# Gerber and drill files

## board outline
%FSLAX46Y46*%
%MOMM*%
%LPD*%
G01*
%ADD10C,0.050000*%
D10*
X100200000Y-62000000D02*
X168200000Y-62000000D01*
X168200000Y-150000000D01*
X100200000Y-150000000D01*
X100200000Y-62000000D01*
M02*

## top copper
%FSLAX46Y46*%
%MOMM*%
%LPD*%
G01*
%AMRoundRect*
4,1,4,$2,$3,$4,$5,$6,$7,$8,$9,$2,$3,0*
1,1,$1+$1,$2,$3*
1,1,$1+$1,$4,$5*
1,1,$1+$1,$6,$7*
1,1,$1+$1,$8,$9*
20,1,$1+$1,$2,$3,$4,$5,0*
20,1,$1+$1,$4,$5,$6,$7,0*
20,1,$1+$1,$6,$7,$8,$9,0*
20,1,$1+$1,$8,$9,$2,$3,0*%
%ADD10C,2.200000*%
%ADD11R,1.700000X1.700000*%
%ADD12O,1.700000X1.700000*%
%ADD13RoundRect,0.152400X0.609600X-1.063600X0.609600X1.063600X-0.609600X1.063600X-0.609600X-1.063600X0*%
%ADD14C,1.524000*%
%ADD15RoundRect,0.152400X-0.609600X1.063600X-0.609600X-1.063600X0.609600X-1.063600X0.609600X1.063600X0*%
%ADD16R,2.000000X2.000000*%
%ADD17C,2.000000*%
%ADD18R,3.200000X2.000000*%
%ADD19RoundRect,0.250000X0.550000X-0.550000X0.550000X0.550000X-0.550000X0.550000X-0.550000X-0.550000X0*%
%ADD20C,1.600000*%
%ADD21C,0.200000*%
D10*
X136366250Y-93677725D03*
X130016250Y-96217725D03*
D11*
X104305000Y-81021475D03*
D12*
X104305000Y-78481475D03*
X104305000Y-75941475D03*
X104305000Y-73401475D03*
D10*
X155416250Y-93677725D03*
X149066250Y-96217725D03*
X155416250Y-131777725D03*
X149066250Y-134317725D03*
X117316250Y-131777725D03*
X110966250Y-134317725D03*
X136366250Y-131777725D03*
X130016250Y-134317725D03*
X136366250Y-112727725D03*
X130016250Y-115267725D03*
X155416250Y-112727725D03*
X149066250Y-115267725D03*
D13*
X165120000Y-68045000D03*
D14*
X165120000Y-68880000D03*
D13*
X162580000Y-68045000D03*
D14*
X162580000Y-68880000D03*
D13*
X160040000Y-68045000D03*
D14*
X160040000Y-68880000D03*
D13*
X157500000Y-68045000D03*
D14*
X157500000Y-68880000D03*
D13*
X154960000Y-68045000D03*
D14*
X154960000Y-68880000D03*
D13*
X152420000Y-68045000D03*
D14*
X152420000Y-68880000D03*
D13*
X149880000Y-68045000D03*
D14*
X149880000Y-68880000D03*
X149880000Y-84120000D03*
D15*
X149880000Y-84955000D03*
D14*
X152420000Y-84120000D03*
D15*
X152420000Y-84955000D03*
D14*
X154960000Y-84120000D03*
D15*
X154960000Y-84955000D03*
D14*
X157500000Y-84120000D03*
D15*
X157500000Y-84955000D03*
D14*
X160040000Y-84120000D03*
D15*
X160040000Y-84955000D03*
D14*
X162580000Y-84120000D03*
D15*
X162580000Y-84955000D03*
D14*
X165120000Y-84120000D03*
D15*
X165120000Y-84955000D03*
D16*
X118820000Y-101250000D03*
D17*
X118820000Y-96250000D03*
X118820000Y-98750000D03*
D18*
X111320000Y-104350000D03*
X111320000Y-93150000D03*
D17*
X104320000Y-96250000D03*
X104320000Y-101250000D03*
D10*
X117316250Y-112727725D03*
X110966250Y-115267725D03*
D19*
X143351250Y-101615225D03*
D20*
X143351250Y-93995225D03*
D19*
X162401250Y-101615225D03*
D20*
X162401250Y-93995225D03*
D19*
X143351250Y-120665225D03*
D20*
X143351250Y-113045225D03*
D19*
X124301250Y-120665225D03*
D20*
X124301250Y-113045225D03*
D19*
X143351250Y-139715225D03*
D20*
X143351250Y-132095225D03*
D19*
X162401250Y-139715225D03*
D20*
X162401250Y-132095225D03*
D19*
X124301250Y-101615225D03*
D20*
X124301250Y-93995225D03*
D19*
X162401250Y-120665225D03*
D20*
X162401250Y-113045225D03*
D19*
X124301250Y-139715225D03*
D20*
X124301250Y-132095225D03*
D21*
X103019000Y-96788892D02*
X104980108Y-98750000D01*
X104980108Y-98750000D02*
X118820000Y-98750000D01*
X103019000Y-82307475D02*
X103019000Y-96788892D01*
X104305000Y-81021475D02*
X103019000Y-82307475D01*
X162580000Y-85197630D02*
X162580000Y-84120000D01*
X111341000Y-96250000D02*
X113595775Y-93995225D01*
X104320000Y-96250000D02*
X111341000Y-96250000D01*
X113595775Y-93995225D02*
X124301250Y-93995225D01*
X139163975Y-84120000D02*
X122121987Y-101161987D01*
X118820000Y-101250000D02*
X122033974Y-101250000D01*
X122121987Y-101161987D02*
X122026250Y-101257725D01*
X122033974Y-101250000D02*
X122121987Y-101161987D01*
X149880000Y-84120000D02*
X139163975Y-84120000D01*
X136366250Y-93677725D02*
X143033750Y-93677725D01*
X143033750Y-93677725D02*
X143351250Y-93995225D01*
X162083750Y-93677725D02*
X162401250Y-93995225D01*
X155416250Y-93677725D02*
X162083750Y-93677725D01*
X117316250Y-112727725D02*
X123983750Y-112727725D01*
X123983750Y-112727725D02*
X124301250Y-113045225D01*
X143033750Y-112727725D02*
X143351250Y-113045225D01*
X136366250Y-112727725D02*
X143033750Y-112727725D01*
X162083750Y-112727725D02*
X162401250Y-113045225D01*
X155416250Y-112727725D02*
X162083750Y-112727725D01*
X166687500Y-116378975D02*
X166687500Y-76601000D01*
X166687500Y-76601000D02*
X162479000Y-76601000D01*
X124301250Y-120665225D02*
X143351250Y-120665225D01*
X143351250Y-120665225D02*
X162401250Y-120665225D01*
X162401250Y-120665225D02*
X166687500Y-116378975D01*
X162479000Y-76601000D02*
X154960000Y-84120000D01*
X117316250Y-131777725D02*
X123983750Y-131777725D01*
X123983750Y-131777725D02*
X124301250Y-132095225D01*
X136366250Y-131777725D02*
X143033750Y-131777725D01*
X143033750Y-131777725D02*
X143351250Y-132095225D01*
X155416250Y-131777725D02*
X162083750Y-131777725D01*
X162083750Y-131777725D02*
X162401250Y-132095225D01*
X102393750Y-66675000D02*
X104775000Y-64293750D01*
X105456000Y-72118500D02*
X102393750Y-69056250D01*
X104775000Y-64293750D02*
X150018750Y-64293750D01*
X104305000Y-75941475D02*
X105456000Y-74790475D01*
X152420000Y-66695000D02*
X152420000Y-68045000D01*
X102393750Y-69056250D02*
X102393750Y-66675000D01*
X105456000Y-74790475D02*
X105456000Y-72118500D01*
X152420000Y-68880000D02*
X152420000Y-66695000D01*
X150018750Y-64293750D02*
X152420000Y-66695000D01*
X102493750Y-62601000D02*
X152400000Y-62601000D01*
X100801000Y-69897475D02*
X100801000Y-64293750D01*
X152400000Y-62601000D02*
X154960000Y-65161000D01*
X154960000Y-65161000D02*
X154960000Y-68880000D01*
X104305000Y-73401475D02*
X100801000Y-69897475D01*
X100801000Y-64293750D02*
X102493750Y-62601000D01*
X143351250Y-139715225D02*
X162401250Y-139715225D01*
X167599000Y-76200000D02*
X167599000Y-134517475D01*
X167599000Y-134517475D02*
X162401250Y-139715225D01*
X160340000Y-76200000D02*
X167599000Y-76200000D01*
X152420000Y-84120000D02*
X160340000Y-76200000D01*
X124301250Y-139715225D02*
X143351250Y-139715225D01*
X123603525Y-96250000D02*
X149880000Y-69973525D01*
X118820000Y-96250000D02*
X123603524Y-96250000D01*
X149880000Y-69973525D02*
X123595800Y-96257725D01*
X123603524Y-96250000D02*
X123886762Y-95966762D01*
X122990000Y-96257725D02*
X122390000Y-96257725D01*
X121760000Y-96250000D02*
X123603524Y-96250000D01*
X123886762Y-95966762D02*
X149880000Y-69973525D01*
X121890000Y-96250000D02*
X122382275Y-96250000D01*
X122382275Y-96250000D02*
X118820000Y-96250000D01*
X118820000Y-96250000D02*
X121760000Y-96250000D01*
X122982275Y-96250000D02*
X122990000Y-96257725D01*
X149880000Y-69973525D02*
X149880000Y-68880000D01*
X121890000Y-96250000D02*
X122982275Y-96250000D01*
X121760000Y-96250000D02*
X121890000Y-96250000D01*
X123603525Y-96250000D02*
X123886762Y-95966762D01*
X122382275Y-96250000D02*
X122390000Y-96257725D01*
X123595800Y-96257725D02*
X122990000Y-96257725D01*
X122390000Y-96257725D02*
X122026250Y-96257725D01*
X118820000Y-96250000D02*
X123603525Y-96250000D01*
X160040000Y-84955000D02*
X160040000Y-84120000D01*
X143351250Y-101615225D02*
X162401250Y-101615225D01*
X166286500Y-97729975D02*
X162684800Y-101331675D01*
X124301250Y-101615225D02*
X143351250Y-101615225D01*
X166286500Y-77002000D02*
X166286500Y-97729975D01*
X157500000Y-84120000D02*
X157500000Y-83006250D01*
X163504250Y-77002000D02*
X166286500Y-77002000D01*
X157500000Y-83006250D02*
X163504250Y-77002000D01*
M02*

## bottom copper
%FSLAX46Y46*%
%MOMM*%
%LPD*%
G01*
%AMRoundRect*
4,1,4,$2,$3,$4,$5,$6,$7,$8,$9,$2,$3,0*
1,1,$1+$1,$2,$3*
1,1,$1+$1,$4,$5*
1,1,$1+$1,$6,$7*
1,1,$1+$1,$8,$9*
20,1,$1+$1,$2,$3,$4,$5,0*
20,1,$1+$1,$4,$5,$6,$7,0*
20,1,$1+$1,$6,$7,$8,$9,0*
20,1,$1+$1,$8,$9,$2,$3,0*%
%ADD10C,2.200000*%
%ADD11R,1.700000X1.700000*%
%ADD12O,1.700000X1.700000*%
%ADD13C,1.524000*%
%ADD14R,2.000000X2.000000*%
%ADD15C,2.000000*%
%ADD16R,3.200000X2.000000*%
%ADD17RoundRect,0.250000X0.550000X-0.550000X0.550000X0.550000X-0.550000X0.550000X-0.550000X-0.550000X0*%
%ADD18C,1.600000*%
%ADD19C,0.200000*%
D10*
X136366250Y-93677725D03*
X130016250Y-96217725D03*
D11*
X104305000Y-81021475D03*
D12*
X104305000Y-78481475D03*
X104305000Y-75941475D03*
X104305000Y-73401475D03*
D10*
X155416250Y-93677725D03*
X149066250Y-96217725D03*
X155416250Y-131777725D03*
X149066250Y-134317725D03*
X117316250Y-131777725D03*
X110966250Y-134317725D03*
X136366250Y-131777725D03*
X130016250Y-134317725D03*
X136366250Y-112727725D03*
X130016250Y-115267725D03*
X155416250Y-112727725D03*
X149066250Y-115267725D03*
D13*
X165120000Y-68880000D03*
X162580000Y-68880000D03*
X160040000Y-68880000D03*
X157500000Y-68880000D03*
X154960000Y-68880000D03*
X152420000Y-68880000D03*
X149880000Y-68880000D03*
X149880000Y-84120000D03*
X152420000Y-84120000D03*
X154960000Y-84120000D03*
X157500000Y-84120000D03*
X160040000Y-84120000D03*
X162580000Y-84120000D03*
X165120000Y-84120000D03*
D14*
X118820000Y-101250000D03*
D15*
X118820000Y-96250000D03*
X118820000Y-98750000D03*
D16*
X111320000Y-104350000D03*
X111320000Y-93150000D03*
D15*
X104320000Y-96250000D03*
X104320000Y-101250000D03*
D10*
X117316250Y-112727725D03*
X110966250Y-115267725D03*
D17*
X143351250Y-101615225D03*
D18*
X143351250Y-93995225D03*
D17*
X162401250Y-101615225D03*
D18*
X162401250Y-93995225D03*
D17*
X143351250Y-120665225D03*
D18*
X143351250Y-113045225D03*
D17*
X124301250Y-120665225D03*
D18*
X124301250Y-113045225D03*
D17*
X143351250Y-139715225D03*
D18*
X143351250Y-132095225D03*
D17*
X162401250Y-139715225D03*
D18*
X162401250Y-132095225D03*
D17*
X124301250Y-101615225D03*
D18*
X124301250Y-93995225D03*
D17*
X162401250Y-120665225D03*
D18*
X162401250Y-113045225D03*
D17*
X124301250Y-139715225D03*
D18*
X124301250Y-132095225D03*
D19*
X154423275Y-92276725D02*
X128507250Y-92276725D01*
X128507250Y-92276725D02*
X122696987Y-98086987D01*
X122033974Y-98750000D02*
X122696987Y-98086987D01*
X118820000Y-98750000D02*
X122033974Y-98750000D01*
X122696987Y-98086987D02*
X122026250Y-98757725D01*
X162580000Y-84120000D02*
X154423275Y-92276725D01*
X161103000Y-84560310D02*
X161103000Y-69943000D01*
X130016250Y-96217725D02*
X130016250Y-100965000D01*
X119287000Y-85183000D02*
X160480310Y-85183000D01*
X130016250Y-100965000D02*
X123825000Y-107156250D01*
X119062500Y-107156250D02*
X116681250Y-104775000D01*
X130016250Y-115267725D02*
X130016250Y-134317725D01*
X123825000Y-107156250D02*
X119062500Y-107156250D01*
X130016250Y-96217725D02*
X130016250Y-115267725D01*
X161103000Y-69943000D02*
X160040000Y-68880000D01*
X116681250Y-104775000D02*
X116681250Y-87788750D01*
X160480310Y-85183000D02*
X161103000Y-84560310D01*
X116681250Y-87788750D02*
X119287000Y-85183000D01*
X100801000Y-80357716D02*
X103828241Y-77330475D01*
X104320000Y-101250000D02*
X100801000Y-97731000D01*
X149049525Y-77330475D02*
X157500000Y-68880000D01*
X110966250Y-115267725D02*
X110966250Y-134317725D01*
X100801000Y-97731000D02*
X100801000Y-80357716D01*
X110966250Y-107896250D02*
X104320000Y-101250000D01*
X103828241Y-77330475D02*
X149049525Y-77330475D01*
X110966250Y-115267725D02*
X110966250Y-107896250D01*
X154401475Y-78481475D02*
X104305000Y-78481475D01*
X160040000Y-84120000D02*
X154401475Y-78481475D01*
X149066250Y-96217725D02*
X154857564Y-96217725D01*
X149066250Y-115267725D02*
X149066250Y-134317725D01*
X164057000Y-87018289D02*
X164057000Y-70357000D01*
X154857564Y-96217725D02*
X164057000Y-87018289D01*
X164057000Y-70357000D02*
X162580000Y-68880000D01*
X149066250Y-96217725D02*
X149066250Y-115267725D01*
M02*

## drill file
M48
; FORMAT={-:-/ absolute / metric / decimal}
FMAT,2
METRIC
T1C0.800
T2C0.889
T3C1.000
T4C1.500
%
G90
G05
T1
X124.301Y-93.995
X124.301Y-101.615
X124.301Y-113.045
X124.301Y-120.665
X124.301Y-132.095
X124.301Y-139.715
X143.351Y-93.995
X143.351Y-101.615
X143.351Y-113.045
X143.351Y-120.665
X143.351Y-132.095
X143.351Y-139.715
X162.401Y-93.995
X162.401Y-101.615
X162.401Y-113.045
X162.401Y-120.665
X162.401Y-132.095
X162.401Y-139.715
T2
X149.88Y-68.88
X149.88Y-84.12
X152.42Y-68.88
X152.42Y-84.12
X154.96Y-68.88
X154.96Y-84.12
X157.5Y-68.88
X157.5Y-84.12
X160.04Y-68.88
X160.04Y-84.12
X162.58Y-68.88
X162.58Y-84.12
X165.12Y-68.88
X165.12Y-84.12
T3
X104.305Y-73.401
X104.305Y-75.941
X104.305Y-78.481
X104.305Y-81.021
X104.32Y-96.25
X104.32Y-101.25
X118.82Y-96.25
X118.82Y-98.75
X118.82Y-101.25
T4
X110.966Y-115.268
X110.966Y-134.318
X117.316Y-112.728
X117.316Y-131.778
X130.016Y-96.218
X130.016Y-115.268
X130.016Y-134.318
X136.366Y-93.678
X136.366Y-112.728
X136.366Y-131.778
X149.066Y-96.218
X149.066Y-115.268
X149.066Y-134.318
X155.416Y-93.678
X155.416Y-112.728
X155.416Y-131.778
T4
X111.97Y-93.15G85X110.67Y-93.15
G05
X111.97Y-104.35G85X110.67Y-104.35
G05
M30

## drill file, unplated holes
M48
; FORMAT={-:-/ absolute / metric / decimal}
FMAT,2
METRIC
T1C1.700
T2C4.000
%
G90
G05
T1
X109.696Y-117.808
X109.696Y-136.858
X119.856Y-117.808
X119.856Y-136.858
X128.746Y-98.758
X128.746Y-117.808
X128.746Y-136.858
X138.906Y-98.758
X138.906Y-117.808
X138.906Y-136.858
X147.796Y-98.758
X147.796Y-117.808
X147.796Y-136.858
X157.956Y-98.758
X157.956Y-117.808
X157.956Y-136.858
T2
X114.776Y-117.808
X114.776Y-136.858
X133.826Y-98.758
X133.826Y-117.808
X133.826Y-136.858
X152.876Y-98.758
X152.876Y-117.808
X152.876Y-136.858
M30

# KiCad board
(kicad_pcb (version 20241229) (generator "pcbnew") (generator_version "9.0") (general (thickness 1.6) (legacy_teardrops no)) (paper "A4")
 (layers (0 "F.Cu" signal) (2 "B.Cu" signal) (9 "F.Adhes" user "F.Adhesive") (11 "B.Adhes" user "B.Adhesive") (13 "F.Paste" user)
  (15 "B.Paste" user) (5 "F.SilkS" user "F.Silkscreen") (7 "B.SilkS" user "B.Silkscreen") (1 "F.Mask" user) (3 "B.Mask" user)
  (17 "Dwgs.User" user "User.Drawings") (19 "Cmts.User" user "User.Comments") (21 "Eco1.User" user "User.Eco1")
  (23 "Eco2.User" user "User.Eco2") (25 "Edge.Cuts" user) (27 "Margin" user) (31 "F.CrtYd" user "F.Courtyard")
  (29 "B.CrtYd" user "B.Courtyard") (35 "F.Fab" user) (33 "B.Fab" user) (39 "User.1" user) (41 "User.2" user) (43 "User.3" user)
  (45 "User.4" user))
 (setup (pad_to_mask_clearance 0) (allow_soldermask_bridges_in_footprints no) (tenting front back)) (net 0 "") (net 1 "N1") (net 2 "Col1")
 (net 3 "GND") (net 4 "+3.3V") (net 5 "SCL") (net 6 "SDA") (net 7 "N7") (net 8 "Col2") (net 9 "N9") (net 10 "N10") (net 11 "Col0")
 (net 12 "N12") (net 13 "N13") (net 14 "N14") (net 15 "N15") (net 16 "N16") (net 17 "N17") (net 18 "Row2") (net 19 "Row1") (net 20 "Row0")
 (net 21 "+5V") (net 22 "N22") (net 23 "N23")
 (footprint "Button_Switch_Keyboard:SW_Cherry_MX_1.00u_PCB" (layer "F.Cu") (at 136.36625 93.677725)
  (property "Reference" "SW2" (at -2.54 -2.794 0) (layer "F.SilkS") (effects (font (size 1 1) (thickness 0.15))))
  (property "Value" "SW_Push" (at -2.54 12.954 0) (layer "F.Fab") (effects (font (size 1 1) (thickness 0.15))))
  (pad "" np_thru_hole circle (at -7.62 5.08) (size 1.7 1.7) (drill 1.7) (layers "*.Cu" "*.Mask"))
  (pad "" np_thru_hole circle (at -2.54 5.08) (size 4 4) (drill 4) (layers "*.Cu" "*.Mask"))
  (pad "" np_thru_hole circle (at 2.54 5.08) (size 1.7 1.7) (drill 1.7) (layers "*.Cu" "*.Mask"))
  (pad "1" thru_hole circle (at 0 0) (size 2.2 2.2) (drill 1.5) (layers "*.Cu" "*.Mask") (remove_unused_layers no) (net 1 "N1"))
  (pad "2" thru_hole circle (at -6.35 2.54) (size 2.2 2.2) (drill 1.5) (layers "*.Cu" "*.Mask") (remove_unused_layers no) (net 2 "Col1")))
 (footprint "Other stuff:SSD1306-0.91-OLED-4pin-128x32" (layer "F.Cu") (at 140.805 83.211475 180)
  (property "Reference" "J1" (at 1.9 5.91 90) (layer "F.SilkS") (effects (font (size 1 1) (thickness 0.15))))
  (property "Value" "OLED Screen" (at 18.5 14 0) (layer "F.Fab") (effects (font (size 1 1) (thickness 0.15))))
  (pad "1" thru_hole rect (at 36.5 2.19 180) (size 1.7 1.7) (drill 1) (layers "*.Cu" "*.Mask") (remove_unused_layers no) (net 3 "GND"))
  (pad "2" thru_hole oval (at 36.5 4.73 180) (size 1.7 1.7) (drill 1) (layers "*.Cu" "*.Mask") (remove_unused_layers no) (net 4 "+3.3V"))
  (pad "3" thru_hole oval (at 36.5 7.27 180) (size 1.7 1.7) (drill 1) (layers "*.Cu" "*.Mask") (remove_unused_layers no) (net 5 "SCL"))
  (pad "4" thru_hole oval (at 36.5 9.81 180) (size 1.7 1.7) (drill 1) (layers "*.Cu" "*.Mask") (remove_unused_layers no) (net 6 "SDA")))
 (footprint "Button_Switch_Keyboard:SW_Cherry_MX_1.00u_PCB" (layer "F.Cu") (at 155.41625 93.677725)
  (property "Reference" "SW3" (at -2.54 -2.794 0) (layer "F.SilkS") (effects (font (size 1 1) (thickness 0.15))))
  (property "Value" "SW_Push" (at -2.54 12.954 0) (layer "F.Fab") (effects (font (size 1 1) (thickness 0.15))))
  (pad "" np_thru_hole circle (at -7.62 5.08) (size 1.7 1.7) (drill 1.7) (layers "*.Cu" "*.Mask"))
  (pad "" np_thru_hole circle (at -2.54 5.08) (size 4 4) (drill 4) (layers "*.Cu" "*.Mask"))
  (pad "" np_thru_hole circle (at 2.54 5.08) (size 1.7 1.7) (drill 1.7) (layers "*.Cu" "*.Mask"))
  (pad "1" thru_hole circle (at 0 0) (size 2.2 2.2) (drill 1.5) (layers "*.Cu" "*.Mask") (remove_unused_layers no) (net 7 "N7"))
  (pad "2" thru_hole circle (at -6.35 2.54) (size 2.2 2.2) (drill 1.5) (layers "*.Cu" "*.Mask") (remove_unused_layers no) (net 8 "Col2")))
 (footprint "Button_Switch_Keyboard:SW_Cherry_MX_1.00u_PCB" (layer "F.Cu") (at 155.41625 131.777725)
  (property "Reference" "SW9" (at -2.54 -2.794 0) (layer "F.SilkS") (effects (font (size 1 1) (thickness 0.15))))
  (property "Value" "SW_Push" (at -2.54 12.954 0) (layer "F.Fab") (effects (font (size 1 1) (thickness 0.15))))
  (pad "" np_thru_hole circle (at -7.62 5.08) (size 1.7 1.7) (drill 1.7) (layers "*.Cu" "*.Mask"))
  (pad "" np_thru_hole circle (at -2.54 5.08) (size 4 4) (drill 4) (layers "*.Cu" "*.Mask"))
  (pad "" np_thru_hole circle (at 2.54 5.08) (size 1.7 1.7) (drill 1.7) (layers "*.Cu" "*.Mask"))
  (pad "1" thru_hole circle (at 0 0) (size 2.2 2.2) (drill 1.5) (layers "*.Cu" "*.Mask") (remove_unused_layers no) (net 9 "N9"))
  (pad "2" thru_hole circle (at -6.35 2.54) (size 2.2 2.2) (drill 1.5) (layers "*.Cu" "*.Mask") (remove_unused_layers no) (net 8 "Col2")))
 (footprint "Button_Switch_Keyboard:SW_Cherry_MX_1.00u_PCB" (layer "F.Cu") (at 117.31625 131.777725)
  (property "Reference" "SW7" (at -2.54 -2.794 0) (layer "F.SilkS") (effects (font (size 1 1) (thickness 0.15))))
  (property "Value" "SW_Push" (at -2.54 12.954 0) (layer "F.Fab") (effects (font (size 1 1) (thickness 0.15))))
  (pad "" np_thru_hole circle (at -7.62 5.08) (size 1.7 1.7) (drill 1.7) (layers "*.Cu" "*.Mask"))
  (pad "" np_thru_hole circle (at -2.54 5.08) (size 4 4) (drill 4) (layers "*.Cu" "*.Mask"))
  (pad "" np_thru_hole circle (at 2.54 5.08) (size 1.7 1.7) (drill 1.7) (layers "*.Cu" "*.Mask"))
  (pad "1" thru_hole circle (at 0 0) (size 2.2 2.2) (drill 1.5) (layers "*.Cu" "*.Mask") (remove_unused_layers no) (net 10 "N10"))
  (pad "2" thru_hole circle (at -6.35 2.54) (size 2.2 2.2) (drill 1.5) (layers "*.Cu" "*.Mask") (remove_unused_layers no) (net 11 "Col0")))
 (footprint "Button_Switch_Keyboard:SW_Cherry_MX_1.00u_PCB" (layer "F.Cu") (at 136.36625 131.777725)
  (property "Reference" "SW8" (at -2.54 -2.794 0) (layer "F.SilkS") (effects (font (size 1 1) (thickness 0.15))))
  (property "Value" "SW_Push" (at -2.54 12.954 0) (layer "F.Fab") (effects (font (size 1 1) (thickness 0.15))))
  (pad "" np_thru_hole circle (at -7.62 5.08) (size 1.7 1.7) (drill 1.7) (layers "*.Cu" "*.Mask"))
  (pad "" np_thru_hole circle (at -2.54 5.08) (size 4 4) (drill 4) (layers "*.Cu" "*.Mask"))
  (pad "" np_thru_hole circle (at 2.54 5.08) (size 1.7 1.7) (drill 1.7) (layers "*.Cu" "*.Mask"))
  (pad "1" thru_hole circle (at 0 0) (size 2.2 2.2) (drill 1.5) (layers "*.Cu" "*.Mask") (remove_unused_layers no) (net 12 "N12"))
  (pad "2" thru_hole circle (at -6.35 2.54) (size 2.2 2.2) (drill 1.5) (layers "*.Cu" "*.Mask") (remove_unused_layers no) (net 2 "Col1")))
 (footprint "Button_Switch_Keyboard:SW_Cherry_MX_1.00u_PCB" (layer "F.Cu") (at 136.36625 112.727725)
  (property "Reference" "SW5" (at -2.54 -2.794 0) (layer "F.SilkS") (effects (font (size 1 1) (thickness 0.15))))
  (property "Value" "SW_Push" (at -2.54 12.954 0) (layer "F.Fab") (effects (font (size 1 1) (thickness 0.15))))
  (pad "" np_thru_hole circle (at -7.62 5.08) (size 1.7 1.7) (drill 1.7) (layers "*.Cu" "*.Mask"))
  (pad "" np_thru_hole circle (at -2.54 5.08) (size 4 4) (drill 4) (layers "*.Cu" "*.Mask"))
  (pad "" np_thru_hole circle (at 2.54 5.08) (size 1.7 1.7) (drill 1.7) (layers "*.Cu" "*.Mask"))
  (pad "1" thru_hole circle (at 0 0) (size 2.2 2.2) (drill 1.5) (layers "*.Cu" "*.Mask") (remove_unused_layers no) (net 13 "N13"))
  (pad "2" thru_hole circle (at -6.35 2.54) (size 2.2 2.2) (drill 1.5) (layers "*.Cu" "*.Mask") (remove_unused_layers no) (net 2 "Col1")))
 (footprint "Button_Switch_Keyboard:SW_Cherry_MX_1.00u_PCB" (layer "F.Cu") (at 155.41625 112.727725)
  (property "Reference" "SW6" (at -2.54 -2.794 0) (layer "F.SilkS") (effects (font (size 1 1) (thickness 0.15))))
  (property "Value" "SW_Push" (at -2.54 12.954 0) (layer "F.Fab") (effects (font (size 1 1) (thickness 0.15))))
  (pad "" np_thru_hole circle (at -7.62 5.08) (size 1.7 1.7) (drill 1.7) (layers "*.Cu" "*.Mask"))
  (pad "" np_thru_hole circle (at -2.54 5.08) (size 4 4) (drill 4) (layers "*.Cu" "*.Mask"))
  (pad "" np_thru_hole circle (at 2.54 5.08) (size 1.7 1.7) (drill 1.7) (layers "*.Cu" "*.Mask"))
  (pad "1" thru_hole circle (at 0 0) (size 2.2 2.2) (drill 1.5) (layers "*.Cu" "*.Mask") (remove_unused_layers no) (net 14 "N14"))
  (pad "2" thru_hole circle (at -6.35 2.54) (size 2.2 2.2) (drill 1.5) (layers "*.Cu" "*.Mask") (remove_unused_layers no) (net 8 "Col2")))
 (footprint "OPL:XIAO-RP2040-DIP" (layer "F.Cu") (at 157.5 76.5 -90)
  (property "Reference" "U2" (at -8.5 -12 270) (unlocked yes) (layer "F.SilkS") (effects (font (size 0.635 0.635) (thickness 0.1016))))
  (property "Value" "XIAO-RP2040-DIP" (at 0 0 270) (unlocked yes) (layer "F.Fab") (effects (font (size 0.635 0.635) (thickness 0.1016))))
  (pad "1" smd roundrect (at -8.455 -7.62 90) (size 2.432 1.524) (layers "F.Cu" "F.Mask") (roundrect_rratio 0.1) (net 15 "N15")
   (thermal_bridge_angle 45))
  (pad "1" thru_hole circle (at -7.62 -7.62 90) (size 1.524 1.524) (drill 0.889) (layers "*.Cu" "*.Mask") (remove_unused_layers no)
   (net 15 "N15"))
  (pad "2" smd roundrect (at -8.455 -5.08 90) (size 2.432 1.524) (layers "F.Cu" "F.Mask") (roundrect_rratio 0.1) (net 8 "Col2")
   (thermal_bridge_angle 45))
  (pad "2" thru_hole circle (at -7.62 -5.08 90) (size 1.524 1.524) (drill 0.889) (layers "*.Cu" "*.Mask") (remove_unused_layers no)
   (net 8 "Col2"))
  (pad "3" smd roundrect (at -8.455 -2.54 90) (size 2.432 1.524) (layers "F.Cu" "F.Mask") (roundrect_rratio 0.1) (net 2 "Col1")
   (thermal_bridge_angle 45))
  (pad "3" thru_hole circle (at -7.62 -2.54 90) (size 1.524 1.524) (drill 0.889) (layers "*.Cu" "*.Mask") (remove_unused_layers no)
   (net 2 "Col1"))
  (pad "4" smd roundrect (at -8.455 0 90) (size 2.432 1.524) (layers "F.Cu" "F.Mask") (roundrect_rratio 0.1) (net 11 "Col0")
   (thermal_bridge_angle 45))
  (pad "4" thru_hole circle (at -7.62 0 90) (size 1.524 1.524) (drill 0.889) (layers "*.Cu" "*.Mask") (remove_unused_layers no)
   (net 11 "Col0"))
  (pad "5" smd roundrect (at -8.455 2.54 90) (size 2.432 1.524) (layers "F.Cu" "F.Mask") (roundrect_rratio 0.1) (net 6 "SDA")
   (thermal_bridge_angle 45))
  (pad "5" thru_hole circle (at -7.62 2.54 90) (size 1.524 1.524) (drill 0.889) (layers "*.Cu" "*.Mask") (remove_unused_layers no)
   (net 6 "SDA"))
  (pad "6" smd roundrect (at -8.455 5.08 90) (size 2.432 1.524) (layers "F.Cu" "F.Mask") (roundrect_rratio 0.1) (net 5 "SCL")
   (thermal_bridge_angle 45))
  (pad "6" thru_hole circle (at -7.62 5.08 90) (size 1.524 1.524) (drill 0.889) (layers "*.Cu" "*.Mask") (remove_unused_layers no)
   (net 5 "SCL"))
  (pad "7" smd roundrect (at -8.455 7.62 90) (size 2.432 1.524) (layers "F.Cu" "F.Mask") (roundrect_rratio 0.1) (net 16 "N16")
   (thermal_bridge_angle 45))
  (pad "7" thru_hole circle (at -7.62 7.62 90) (size 1.524 1.524) (drill 0.889) (layers "*.Cu" "*.Mask") (remove_unused_layers no)
   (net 16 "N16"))
  (pad "8" thru_hole circle (at 7.62 7.62 270) (size 1.524 1.524) (drill 0.889) (layers "*.Cu" "*.Mask") (remove_unused_layers no)
   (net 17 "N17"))
  (pad "8" smd roundrect (at 8.455 7.62 270) (size 2.432 1.524) (layers "F.Cu" "F.Mask") (roundrect_rratio 0.1) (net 17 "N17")
   (thermal_bridge_angle 45))
  (pad "9" thru_hole circle (at 7.62 5.08 270) (size 1.524 1.524) (drill 0.889) (layers "*.Cu" "*.Mask") (remove_unused_layers no)
   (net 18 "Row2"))
  (pad "9" smd roundrect (at 8.455 5.08 270) (size 2.432 1.524) (layers "F.Cu" "F.Mask") (roundrect_rratio 0.1) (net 18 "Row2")
   (thermal_bridge_angle 45))
  (pad "10" thru_hole circle (at 7.62 2.54 270) (size 1.524 1.524) (drill 0.889) (layers "*.Cu" "*.Mask") (remove_unused_layers no)
   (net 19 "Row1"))
  (pad "10" smd roundrect (at 8.455 2.54 270) (size 2.432 1.524) (layers "F.Cu" "F.Mask") (roundrect_rratio 0.1) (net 19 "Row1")
   (thermal_bridge_angle 45))
  (pad "11" thru_hole circle (at 7.62 0 270) (size 1.524 1.524) (drill 0.889) (layers "*.Cu" "*.Mask") (remove_unused_layers no)
   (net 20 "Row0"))
  (pad "11" smd roundrect (at 8.455 0 270) (size 2.432 1.524) (layers "F.Cu" "F.Mask") (roundrect_rratio 0.1) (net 20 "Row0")
   (thermal_bridge_angle 45))
  (pad "12" thru_hole circle (at 7.62 -2.54 270) (size 1.524 1.524) (drill 0.889) (layers "*.Cu" "*.Mask") (remove_unused_layers no)
   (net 4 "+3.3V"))
  (pad "12" smd roundrect (at 8.455 -2.54 270) (size 2.432 1.524) (layers "F.Cu" "F.Mask") (roundrect_rratio 0.1) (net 4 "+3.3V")
   (thermal_bridge_angle 45))
  (pad "13" thru_hole circle (at 7.62 -5.08 270) (size 1.524 1.524) (drill 0.889) (layers "*.Cu" "*.Mask") (remove_unused_layers no)
   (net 3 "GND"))
  (pad "13" smd roundrect (at 8.455 -5.08 270) (size 2.432 1.524) (layers "F.Cu" "F.Mask") (roundrect_rratio 0.1) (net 3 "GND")
   (thermal_bridge_angle 45))
  (pad "14" thru_hole circle (at 7.62 -7.62 270) (size 1.524 1.524) (drill 0.889) (layers "*.Cu" "*.Mask") (remove_unused_layers no)
   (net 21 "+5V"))
  (pad "14" smd roundrect (at 8.455 -7.62 270) (size 2.432 1.524) (layers "F.Cu" "F.Mask") (roundrect_rratio 0.1) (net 21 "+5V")
   (thermal_bridge_angle 45)))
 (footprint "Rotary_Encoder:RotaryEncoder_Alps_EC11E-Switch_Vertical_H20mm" (layer "F.Cu") (at 118.82 101.25 180)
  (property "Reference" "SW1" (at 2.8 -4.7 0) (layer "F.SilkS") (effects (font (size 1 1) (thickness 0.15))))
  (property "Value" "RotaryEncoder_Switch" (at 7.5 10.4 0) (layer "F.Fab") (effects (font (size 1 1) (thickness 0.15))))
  (pad "A" thru_hole rect (at 0 0 180) (size 2 2) (drill 1) (layers "*.Cu" "*.Mask") (remove_unused_layers no) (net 17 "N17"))
  (pad "B" thru_hole circle (at 0 5 180) (size 2 2) (drill 1) (layers "*.Cu" "*.Mask") (remove_unused_layers no) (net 16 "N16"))
  (pad "C" thru_hole circle (at 0 2.5 180) (size 2 2) (drill 1) (layers "*.Cu" "*.Mask") (remove_unused_layers no) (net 3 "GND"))
  (pad "MP" thru_hole rect (at 7.5 -3.1 180) (size 3.2 2) (drill oval 2.8 1.5) (layers "*.Cu" "*.Mask") (remove_unused_layers no))
  (pad "MP" thru_hole rect (at 7.5 8.1 180) (size 3.2 2) (drill oval 2.8 1.5) (layers "*.Cu" "*.Mask") (remove_unused_layers no))
  (pad "S1" thru_hole circle (at 14.5 5 180) (size 2 2) (drill 1) (layers "*.Cu" "*.Mask") (remove_unused_layers no) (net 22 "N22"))
  (pad "S2" thru_hole circle (at 14.5 0 180) (size 2 2) (drill 1) (layers "*.Cu" "*.Mask") (remove_unused_layers no) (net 11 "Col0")))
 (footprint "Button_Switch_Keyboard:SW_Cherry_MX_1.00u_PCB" (layer "F.Cu") (at 117.31625 112.727725)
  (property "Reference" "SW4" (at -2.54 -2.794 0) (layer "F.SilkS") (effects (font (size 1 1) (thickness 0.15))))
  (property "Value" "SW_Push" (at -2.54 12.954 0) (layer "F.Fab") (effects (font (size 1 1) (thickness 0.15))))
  (pad "" np_thru_hole circle (at -7.62 5.08) (size 1.7 1.7) (drill 1.7) (layers "*.Cu" "*.Mask"))
  (pad "" np_thru_hole circle (at -2.54 5.08) (size 4 4) (drill 4) (layers "*.Cu" "*.Mask"))
  (pad "" np_thru_hole circle (at 2.54 5.08) (size 1.7 1.7) (drill 1.7) (layers "*.Cu" "*.Mask"))
  (pad "1" thru_hole circle (at 0 0) (size 2.2 2.2) (drill 1.5) (layers "*.Cu" "*.Mask") (remove_unused_layers no) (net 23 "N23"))
  (pad "2" thru_hole circle (at -6.35 2.54) (size 2.2 2.2) (drill 1.5) (layers "*.Cu" "*.Mask") (remove_unused_layers no) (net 11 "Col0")))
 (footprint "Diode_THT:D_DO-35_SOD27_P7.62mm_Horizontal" (layer "B.Cu") (at 143.35125 101.615225 90)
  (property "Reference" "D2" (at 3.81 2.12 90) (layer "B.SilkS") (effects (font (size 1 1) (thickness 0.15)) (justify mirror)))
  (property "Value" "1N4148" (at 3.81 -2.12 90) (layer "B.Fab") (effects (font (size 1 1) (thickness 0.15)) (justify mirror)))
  (pad "1" thru_hole roundrect (at 0 0 90) (size 1.6 1.6) (drill 0.8) (layers "*.Cu" "*.Mask") (remove_unused_layers no)
   (roundrect_rratio 0.15625) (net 20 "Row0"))
  (pad "2" thru_hole circle (at 7.62 0 90) (size 1.6 1.6) (drill 0.8) (layers "*.Cu" "*.Mask") (remove_unused_layers no) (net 1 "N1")))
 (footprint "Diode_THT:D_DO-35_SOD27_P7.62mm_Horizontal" (layer "B.Cu") (at 162.40125 101.615225 90)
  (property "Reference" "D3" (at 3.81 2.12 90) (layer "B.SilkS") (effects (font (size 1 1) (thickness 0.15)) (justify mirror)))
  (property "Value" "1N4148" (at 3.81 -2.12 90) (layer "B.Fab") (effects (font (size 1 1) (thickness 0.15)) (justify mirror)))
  (pad "1" thru_hole roundrect (at 0 0 90) (size 1.6 1.6) (drill 0.8) (layers "*.Cu" "*.Mask") (remove_unused_layers no)
   (roundrect_rratio 0.15625) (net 20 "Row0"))
  (pad "2" thru_hole circle (at 7.62 0 90) (size 1.6 1.6) (drill 0.8) (layers "*.Cu" "*.Mask") (remove_unused_layers no) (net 7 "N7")))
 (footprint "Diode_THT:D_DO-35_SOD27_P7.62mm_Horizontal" (layer "B.Cu") (at 143.35125 120.665225 90)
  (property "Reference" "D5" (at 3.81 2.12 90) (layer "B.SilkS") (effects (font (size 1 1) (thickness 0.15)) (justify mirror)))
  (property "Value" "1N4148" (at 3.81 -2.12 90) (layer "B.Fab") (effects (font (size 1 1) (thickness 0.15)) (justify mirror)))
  (pad "1" thru_hole roundrect (at 0 0 90) (size 1.6 1.6) (drill 0.8) (layers "*.Cu" "*.Mask") (remove_unused_layers no)
   (roundrect_rratio 0.15625) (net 19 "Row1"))
  (pad "2" thru_hole circle (at 7.62 0 90) (size 1.6 1.6) (drill 0.8) (layers "*.Cu" "*.Mask") (remove_unused_layers no) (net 13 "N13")))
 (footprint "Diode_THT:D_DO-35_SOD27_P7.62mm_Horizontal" (layer "B.Cu") (at 124.30125 120.665225 90)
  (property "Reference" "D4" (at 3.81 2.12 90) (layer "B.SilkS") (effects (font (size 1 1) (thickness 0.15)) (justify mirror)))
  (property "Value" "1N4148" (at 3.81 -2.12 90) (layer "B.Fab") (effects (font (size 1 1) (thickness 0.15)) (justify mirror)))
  (pad "1" thru_hole roundrect (at 0 0 90) (size 1.6 1.6) (drill 0.8) (layers "*.Cu" "*.Mask") (remove_unused_layers no)
   (roundrect_rratio 0.15625) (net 19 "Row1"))
  (pad "2" thru_hole circle (at 7.62 0 90) (size 1.6 1.6) (drill 0.8) (layers "*.Cu" "*.Mask") (remove_unused_layers no) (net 23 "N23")))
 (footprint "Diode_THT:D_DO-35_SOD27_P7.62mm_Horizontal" (layer "B.Cu") (at 143.35125 139.715225 90)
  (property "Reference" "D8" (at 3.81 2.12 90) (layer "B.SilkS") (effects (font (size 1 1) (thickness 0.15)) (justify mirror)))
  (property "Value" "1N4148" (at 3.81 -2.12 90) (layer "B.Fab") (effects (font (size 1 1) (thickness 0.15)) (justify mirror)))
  (pad "1" thru_hole roundrect (at 0 0 90) (size 1.6 1.6) (drill 0.8) (layers "*.Cu" "*.Mask") (remove_unused_layers no)
   (roundrect_rratio 0.15625) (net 18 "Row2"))
  (pad "2" thru_hole circle (at 7.62 0 90) (size 1.6 1.6) (drill 0.8) (layers "*.Cu" "*.Mask") (remove_unused_layers no) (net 12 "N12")))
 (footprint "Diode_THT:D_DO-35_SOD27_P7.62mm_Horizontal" (layer "B.Cu") (at 162.40125 139.715225 90)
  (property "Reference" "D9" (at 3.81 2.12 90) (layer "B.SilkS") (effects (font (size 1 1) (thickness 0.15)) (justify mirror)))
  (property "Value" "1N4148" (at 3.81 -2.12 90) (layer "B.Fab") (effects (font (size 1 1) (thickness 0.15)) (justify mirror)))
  (pad "1" thru_hole roundrect (at 0 0 90) (size 1.6 1.6) (drill 0.8) (layers "*.Cu" "*.Mask") (remove_unused_layers no)
   (roundrect_rratio 0.15625) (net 18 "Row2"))
  (pad "2" thru_hole circle (at 7.62 0 90) (size 1.6 1.6) (drill 0.8) (layers "*.Cu" "*.Mask") (remove_unused_layers no) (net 9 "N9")))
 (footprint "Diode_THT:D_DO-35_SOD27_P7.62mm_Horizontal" (layer "B.Cu") (at 124.30125 101.615225 90)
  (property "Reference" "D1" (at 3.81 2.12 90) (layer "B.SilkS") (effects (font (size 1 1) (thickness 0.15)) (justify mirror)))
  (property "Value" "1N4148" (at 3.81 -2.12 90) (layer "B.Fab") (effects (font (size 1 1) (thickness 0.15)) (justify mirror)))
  (pad "1" thru_hole roundrect (at 0 0 90) (size 1.6 1.6) (drill 0.8) (layers "*.Cu" "*.Mask") (remove_unused_layers no)
   (roundrect_rratio 0.15625) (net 20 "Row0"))
  (pad "2" thru_hole circle (at 7.62 0 90) (size 1.6 1.6) (drill 0.8) (layers "*.Cu" "*.Mask") (remove_unused_layers no) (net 22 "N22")))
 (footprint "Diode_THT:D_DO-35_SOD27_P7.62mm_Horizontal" (layer "B.Cu") (at 162.40125 120.665225 90)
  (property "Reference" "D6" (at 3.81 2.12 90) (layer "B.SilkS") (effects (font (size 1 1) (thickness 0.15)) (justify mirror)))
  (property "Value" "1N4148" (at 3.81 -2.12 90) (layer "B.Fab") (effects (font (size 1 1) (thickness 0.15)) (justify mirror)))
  (pad "1" thru_hole roundrect (at 0 0 90) (size 1.6 1.6) (drill 0.8) (layers "*.Cu" "*.Mask") (remove_unused_layers no)
   (roundrect_rratio 0.15625) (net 19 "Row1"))
  (pad "2" thru_hole circle (at 7.62 0 90) (size 1.6 1.6) (drill 0.8) (layers "*.Cu" "*.Mask") (remove_unused_layers no) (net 14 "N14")))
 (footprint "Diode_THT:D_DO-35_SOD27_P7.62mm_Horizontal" (layer "B.Cu") (at 124.30125 139.715225 90)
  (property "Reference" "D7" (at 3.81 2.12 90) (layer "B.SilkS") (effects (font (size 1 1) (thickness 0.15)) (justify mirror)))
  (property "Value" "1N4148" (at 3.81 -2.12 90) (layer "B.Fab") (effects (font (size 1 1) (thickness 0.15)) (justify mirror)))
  (pad "1" thru_hole roundrect (at 0 0 90) (size 1.6 1.6) (drill 0.8) (layers "*.Cu" "*.Mask") (remove_unused_layers no)
   (roundrect_rratio 0.15625) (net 18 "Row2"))
  (pad "2" thru_hole circle (at 7.62 0 90) (size 1.6 1.6) (drill 0.8) (layers "*.Cu" "*.Mask") (remove_unused_layers no) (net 10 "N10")))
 (gr_rect (start 100.2 62) (end 168.2 150) (stroke (width 0.05) (type default)) (fill no) (layer "Edge.Cuts"))
 (segment (start 103.019 96.788892) (end 104.980108 98.75) (width 0.2) (layer "F.Cu") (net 3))
 (segment (start 104.980108 98.75) (end 118.82 98.75) (width 0.2) (layer "F.Cu") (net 3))
 (segment (start 103.019 82.307475) (end 103.019 96.788892) (width 0.2) (layer "F.Cu") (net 3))
 (segment (start 104.305 81.021475) (end 103.019 82.307475) (width 0.2) (layer "F.Cu") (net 3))
 (segment (start 162.58 85.19763) (end 162.58 84.12) (width 0.2) (layer "F.Cu") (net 3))
 (segment (start 154.423275 92.276725) (end 128.50725 92.276725) (width 0.2) (layer "B.Cu") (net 3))
 (segment (start 128.50725 92.276725) (end 122.696987 98.086987) (width 0.2) (layer "B.Cu") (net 3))
 (segment (start 122.033974 98.75) (end 122.696987 98.086987) (width 0.2) (layer "B.Cu") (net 3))
 (segment (start 118.82 98.75) (end 122.033974 98.75) (width 0.2) (layer "B.Cu") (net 3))
 (segment (start 122.696987 98.086987) (end 122.02625 98.757725) (width 0.2) (layer "B.Cu") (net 3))
 (segment (start 162.58 84.12) (end 154.423275 92.276725) (width 0.2) (layer "B.Cu") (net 3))
 (segment (start 111.341 96.25) (end 113.595775 93.995225) (width 0.2) (layer "F.Cu") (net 22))
 (segment (start 104.32 96.25) (end 111.341 96.25) (width 0.2) (layer "F.Cu") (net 22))
 (segment (start 113.595775 93.995225) (end 124.30125 93.995225) (width 0.2) (layer "F.Cu") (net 22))
 (segment (start 139.163975 84.12) (end 122.121987 101.161987) (width 0.2) (layer "F.Cu") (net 17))
 (segment (start 118.82 101.25) (end 122.033974 101.25) (width 0.2) (layer "F.Cu") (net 17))
 (segment (start 122.121987 101.161987) (end 122.02625 101.257725) (width 0.2) (layer "F.Cu") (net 17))
 (segment (start 122.033974 101.25) (end 122.121987 101.161987) (width 0.2) (layer "F.Cu") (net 17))
 (segment (start 149.88 84.12) (end 139.163975 84.12) (width 0.2) (layer "F.Cu") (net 17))
 (segment (start 136.36625 93.677725) (end 143.03375 93.677725) (width 0.2) (layer "F.Cu") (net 1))
 (segment (start 143.03375 93.677725) (end 143.35125 93.995225) (width 0.2) (layer "F.Cu") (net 1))
 (segment (start 162.08375 93.677725) (end 162.40125 93.995225) (width 0.2) (layer "F.Cu") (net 7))
 (segment (start 155.41625 93.677725) (end 162.08375 93.677725) (width 0.2) (layer "F.Cu") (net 7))
 (segment (start 117.31625 112.727725) (end 123.98375 112.727725) (width 0.2) (layer "F.Cu") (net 23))
 (segment (start 123.98375 112.727725) (end 124.30125 113.045225) (width 0.2) (layer "F.Cu") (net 23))
 (segment (start 161.103 84.56031) (end 161.103 69.943) (width 0.2) (layer "B.Cu") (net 2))
 (segment (start 130.01625 96.217725) (end 130.01625 100.965) (width 0.2) (layer "B.Cu") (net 2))
 (segment (start 119.287 85.183) (end 160.48031 85.183) (width 0.2) (layer "B.Cu") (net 2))
 (segment (start 130.01625 100.965) (end 123.825 107.15625) (width 0.2) (layer "B.Cu") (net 2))
 (segment (start 119.0625 107.15625) (end 116.68125 104.775) (width 0.2) (layer "B.Cu") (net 2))
 (segment (start 130.01625 115.267725) (end 130.01625 134.317725) (width 0.2) (layer "B.Cu") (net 2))
 (segment (start 123.825 107.15625) (end 119.0625 107.15625) (width 0.2) (layer "B.Cu") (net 2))
 (segment (start 130.01625 96.217725) (end 130.01625 115.267725) (width 0.2) (layer "B.Cu") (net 2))
 (segment (start 161.103 69.943) (end 160.04 68.88) (width 0.2) (layer "B.Cu") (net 2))
 (segment (start 116.68125 104.775) (end 116.68125 87.78875) (width 0.2) (layer "B.Cu") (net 2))
 (segment (start 160.48031 85.183) (end 161.103 84.56031) (width 0.2) (layer "B.Cu") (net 2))
 (segment (start 116.68125 87.78875) (end 119.287 85.183) (width 0.2) (layer "B.Cu") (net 2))
 (segment (start 143.03375 112.727725) (end 143.35125 113.045225) (width 0.2) (layer "F.Cu") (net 13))
 (segment (start 136.36625 112.727725) (end 143.03375 112.727725) (width 0.2) (layer "F.Cu") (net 13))
 (segment (start 162.08375 112.727725) (end 162.40125 113.045225) (width 0.2) (layer "F.Cu") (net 14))
 (segment (start 155.41625 112.727725) (end 162.08375 112.727725) (width 0.2) (layer "F.Cu") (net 14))
 (segment (start 166.6875 116.378975) (end 166.6875 76.601) (width 0.2) (layer "F.Cu") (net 19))
 (segment (start 166.6875 76.601) (end 162.479 76.601) (width 0.2) (layer "F.Cu") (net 19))
 (segment (start 124.30125 120.665225) (end 143.35125 120.665225) (width 0.2) (layer "F.Cu") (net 19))
 (segment (start 143.35125 120.665225) (end 162.40125 120.665225) (width 0.2) (layer "F.Cu") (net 19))
 (segment (start 162.40125 120.665225) (end 166.6875 116.378975) (width 0.2) (layer "F.Cu") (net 19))
 (segment (start 162.479 76.601) (end 154.96 84.12) (width 0.2) (layer "F.Cu") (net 19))
 (segment (start 117.31625 131.777725) (end 123.98375 131.777725) (width 0.2) (layer "F.Cu") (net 10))
 (segment (start 123.98375 131.777725) (end 124.30125 132.095225) (width 0.2) (layer "F.Cu") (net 10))
 (segment (start 136.36625 131.777725) (end 143.03375 131.777725) (width 0.2) (layer "F.Cu") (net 12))
 (segment (start 143.03375 131.777725) (end 143.35125 132.095225) (width 0.2) (layer "F.Cu") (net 12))
 (segment (start 155.41625 131.777725) (end 162.08375 131.777725) (width 0.2) (layer "F.Cu") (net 9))
 (segment (start 162.08375 131.777725) (end 162.40125 132.095225) (width 0.2) (layer "F.Cu") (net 9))
 (segment (start 102.39375 66.675) (end 104.775 64.29375) (width 0.2) (layer "F.Cu") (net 5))
 (segment (start 105.456 72.1185) (end 102.39375 69.05625) (width 0.2) (layer "F.Cu") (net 5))
 (segment (start 104.775 64.29375) (end 150.01875 64.29375) (width 0.2) (layer "F.Cu") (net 5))
 (segment (start 104.305 75.941475) (end 105.456 74.790475) (width 0.2) (layer "F.Cu") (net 5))
 (segment (start 152.42 66.695) (end 152.42 68.045) (width 0.2) (layer "F.Cu") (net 5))
 (segment (start 102.39375 69.05625) (end 102.39375 66.675) (width 0.2) (layer "F.Cu") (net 5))
 (segment (start 105.456 74.790475) (end 105.456 72.1185) (width 0.2) (layer "F.Cu") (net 5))
 (segment (start 152.42 68.88) (end 152.42 66.695) (width 0.2) (layer "F.Cu") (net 5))
 (segment (start 150.01875 64.29375) (end 152.42 66.695) (width 0.2) (layer "F.Cu") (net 5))
 (segment (start 102.49375 62.601) (end 152.4 62.601) (width 0.2) (layer "F.Cu") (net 6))
 (segment (start 100.801 69.897475) (end 100.801 64.29375) (width 0.2) (layer "F.Cu") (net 6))
 (segment (start 152.4 62.601) (end 154.96 65.161) (width 0.2) (layer "F.Cu") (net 6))
 (segment (start 154.96 65.161) (end 154.96 68.88) (width 0.2) (layer "F.Cu") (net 6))
 (segment (start 104.305 73.401475) (end 100.801 69.897475) (width 0.2) (layer "F.Cu") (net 6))
 (segment (start 100.801 64.29375) (end 102.49375 62.601) (width 0.2) (layer "F.Cu") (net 6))
 (segment (start 143.35125 139.715225) (end 162.40125 139.715225) (width 0.2) (layer "F.Cu") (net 18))
 (segment (start 167.599 76.2) (end 167.599 134.517475) (width 0.2) (layer "F.Cu") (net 18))
 (segment (start 167.599 134.517475) (end 162.40125 139.715225) (width 0.2) (layer "F.Cu") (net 18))
 (segment (start 160.34 76.2) (end 167.599 76.2) (width 0.2) (layer "F.Cu") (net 18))
 (segment (start 152.42 84.12) (end 160.34 76.2) (width 0.2) (layer "F.Cu") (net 18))
 (segment (start 124.30125 139.715225) (end 143.35125 139.715225) (width 0.2) (layer "F.Cu") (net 18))
 (segment (start 100.801 80.357716) (end 103.828241 77.330475) (width 0.2) (layer "B.Cu") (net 11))
 (segment (start 104.32 101.25) (end 100.801 97.731) (width 0.2) (layer "B.Cu") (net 11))
 (segment (start 149.049525 77.330475) (end 157.5 68.88) (width 0.2) (layer "B.Cu") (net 11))
 (segment (start 110.96625 115.267725) (end 110.96625 134.317725) (width 0.2) (layer "B.Cu") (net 11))
 (segment (start 100.801 97.731) (end 100.801 80.357716) (width 0.2) (layer "B.Cu") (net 11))
 (segment (start 110.96625 107.89625) (end 104.32 101.25) (width 0.2) (layer "B.Cu") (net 11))
 (segment (start 103.828241 77.330475) (end 149.049525 77.330475) (width 0.2) (layer "B.Cu") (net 11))
 (segment (start 110.96625 115.267725) (end 110.96625 107.89625) (width 0.2) (layer "B.Cu") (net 11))
 (segment (start 123.603525 96.25) (end 149.88 69.973525) (width 0.2) (layer "F.Cu") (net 16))
 (segment (start 118.82 96.25) (end 123.603524 96.25) (width 0.2) (layer "F.Cu") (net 16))
 (segment (start 149.88 69.973525) (end 123.5958 96.257725) (width 0.2) (layer "F.Cu") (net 16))
 (segment (start 123.603524 96.25) (end 123.886762 95.966762) (width 0.2) (layer "F.Cu") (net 16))
 (segment (start 122.99 96.257725) (end 122.39 96.257725) (width 0.2) (layer "F.Cu") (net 16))
 (segment (start 121.76 96.25) (end 123.603524 96.25) (width 0.2) (layer "F.Cu") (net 16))
 (segment (start 123.886762 95.966762) (end 149.88 69.973525) (width 0.2) (layer "F.Cu") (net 16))
 (segment (start 121.89 96.25) (end 122.382275 96.25) (width 0.2) (layer "F.Cu") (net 16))
 (segment (start 122.382275 96.25) (end 118.82 96.25) (width 0.2) (layer "F.Cu") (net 16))
 (segment (start 118.82 96.25) (end 121.76 96.25) (width 0.2) (layer "F.Cu") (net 16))
 (segment (start 122.982275 96.25) (end 122.99 96.257725) (width 0.2) (layer "F.Cu") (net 16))
 (segment (start 149.88 69.973525) (end 149.88 68.88) (width 0.2) (layer "F.Cu") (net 16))
 (segment (start 121.89 96.25) (end 122.982275 96.25) (width 0.2) (layer "F.Cu") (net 16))
 (segment (start 121.76 96.25) (end 121.89 96.25) (width 0.2) (layer "F.Cu") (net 16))
 (segment (start 123.603525 96.25) (end 123.886762 95.966762) (width 0.2) (layer "F.Cu") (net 16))
 (segment (start 122.382275 96.25) (end 122.39 96.257725) (width 0.2) (layer "F.Cu") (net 16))
 (segment (start 123.5958 96.257725) (end 122.99 96.257725) (width 0.2) (layer "F.Cu") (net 16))
 (segment (start 122.39 96.257725) (end 122.02625 96.257725) (width 0.2) (layer "F.Cu") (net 16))
 (segment (start 118.82 96.25) (end 123.603525 96.25) (width 0.2) (layer "F.Cu") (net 16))
 (segment (start 160.04 84.955) (end 160.04 84.12) (width 0.2) (layer "F.Cu") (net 4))
 (segment (start 154.401475 78.481475) (end 104.305 78.481475) (width 0.2) (layer "B.Cu") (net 4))
 (segment (start 160.04 84.12) (end 154.401475 78.481475) (width 0.2) (layer "B.Cu") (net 4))
 (segment (start 143.35125 101.615225) (end 162.40125 101.615225) (width 0.2) (layer "F.Cu") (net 20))
 (segment (start 166.2865 97.729975) (end 162.6848 101.331675) (width 0.2) (layer "F.Cu") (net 20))
 (segment (start 124.30125 101.615225) (end 143.35125 101.615225) (width 0.2) (layer "F.Cu") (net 20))
 (segment (start 166.2865 77.002) (end 166.2865 97.729975) (width 0.2) (layer "F.Cu") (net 20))
 (segment (start 157.5 84.12) (end 157.5 83.00625) (width 0.2) (layer "F.Cu") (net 20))
 (segment (start 163.50425 77.002) (end 166.2865 77.002) (width 0.2) (layer "F.Cu") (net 20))
 (segment (start 157.5 83.00625) (end 163.50425 77.002) (width 0.2) (layer "F.Cu") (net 20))
 (segment (start 149.06625 96.217725) (end 154.857564 96.217725) (width 0.2) (layer "B.Cu") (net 8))
 (segment (start 149.06625 115.267725) (end 149.06625 134.317725) (width 0.2) (layer "B.Cu") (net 8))
 (segment (start 164.057 87.018289) (end 164.057 70.357) (width 0.2) (layer "B.Cu") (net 8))
 (segment (start 154.857564 96.217725) (end 164.057 87.018289) (width 0.2) (layer "B.Cu") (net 8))
 (segment (start 164.057 70.357) (end 162.58 68.88) (width 0.2) (layer "B.Cu") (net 8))
 (segment (start 149.06625 96.217725) (end 149.06625 115.267725) (width 0.2) (layer "B.Cu") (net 8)))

